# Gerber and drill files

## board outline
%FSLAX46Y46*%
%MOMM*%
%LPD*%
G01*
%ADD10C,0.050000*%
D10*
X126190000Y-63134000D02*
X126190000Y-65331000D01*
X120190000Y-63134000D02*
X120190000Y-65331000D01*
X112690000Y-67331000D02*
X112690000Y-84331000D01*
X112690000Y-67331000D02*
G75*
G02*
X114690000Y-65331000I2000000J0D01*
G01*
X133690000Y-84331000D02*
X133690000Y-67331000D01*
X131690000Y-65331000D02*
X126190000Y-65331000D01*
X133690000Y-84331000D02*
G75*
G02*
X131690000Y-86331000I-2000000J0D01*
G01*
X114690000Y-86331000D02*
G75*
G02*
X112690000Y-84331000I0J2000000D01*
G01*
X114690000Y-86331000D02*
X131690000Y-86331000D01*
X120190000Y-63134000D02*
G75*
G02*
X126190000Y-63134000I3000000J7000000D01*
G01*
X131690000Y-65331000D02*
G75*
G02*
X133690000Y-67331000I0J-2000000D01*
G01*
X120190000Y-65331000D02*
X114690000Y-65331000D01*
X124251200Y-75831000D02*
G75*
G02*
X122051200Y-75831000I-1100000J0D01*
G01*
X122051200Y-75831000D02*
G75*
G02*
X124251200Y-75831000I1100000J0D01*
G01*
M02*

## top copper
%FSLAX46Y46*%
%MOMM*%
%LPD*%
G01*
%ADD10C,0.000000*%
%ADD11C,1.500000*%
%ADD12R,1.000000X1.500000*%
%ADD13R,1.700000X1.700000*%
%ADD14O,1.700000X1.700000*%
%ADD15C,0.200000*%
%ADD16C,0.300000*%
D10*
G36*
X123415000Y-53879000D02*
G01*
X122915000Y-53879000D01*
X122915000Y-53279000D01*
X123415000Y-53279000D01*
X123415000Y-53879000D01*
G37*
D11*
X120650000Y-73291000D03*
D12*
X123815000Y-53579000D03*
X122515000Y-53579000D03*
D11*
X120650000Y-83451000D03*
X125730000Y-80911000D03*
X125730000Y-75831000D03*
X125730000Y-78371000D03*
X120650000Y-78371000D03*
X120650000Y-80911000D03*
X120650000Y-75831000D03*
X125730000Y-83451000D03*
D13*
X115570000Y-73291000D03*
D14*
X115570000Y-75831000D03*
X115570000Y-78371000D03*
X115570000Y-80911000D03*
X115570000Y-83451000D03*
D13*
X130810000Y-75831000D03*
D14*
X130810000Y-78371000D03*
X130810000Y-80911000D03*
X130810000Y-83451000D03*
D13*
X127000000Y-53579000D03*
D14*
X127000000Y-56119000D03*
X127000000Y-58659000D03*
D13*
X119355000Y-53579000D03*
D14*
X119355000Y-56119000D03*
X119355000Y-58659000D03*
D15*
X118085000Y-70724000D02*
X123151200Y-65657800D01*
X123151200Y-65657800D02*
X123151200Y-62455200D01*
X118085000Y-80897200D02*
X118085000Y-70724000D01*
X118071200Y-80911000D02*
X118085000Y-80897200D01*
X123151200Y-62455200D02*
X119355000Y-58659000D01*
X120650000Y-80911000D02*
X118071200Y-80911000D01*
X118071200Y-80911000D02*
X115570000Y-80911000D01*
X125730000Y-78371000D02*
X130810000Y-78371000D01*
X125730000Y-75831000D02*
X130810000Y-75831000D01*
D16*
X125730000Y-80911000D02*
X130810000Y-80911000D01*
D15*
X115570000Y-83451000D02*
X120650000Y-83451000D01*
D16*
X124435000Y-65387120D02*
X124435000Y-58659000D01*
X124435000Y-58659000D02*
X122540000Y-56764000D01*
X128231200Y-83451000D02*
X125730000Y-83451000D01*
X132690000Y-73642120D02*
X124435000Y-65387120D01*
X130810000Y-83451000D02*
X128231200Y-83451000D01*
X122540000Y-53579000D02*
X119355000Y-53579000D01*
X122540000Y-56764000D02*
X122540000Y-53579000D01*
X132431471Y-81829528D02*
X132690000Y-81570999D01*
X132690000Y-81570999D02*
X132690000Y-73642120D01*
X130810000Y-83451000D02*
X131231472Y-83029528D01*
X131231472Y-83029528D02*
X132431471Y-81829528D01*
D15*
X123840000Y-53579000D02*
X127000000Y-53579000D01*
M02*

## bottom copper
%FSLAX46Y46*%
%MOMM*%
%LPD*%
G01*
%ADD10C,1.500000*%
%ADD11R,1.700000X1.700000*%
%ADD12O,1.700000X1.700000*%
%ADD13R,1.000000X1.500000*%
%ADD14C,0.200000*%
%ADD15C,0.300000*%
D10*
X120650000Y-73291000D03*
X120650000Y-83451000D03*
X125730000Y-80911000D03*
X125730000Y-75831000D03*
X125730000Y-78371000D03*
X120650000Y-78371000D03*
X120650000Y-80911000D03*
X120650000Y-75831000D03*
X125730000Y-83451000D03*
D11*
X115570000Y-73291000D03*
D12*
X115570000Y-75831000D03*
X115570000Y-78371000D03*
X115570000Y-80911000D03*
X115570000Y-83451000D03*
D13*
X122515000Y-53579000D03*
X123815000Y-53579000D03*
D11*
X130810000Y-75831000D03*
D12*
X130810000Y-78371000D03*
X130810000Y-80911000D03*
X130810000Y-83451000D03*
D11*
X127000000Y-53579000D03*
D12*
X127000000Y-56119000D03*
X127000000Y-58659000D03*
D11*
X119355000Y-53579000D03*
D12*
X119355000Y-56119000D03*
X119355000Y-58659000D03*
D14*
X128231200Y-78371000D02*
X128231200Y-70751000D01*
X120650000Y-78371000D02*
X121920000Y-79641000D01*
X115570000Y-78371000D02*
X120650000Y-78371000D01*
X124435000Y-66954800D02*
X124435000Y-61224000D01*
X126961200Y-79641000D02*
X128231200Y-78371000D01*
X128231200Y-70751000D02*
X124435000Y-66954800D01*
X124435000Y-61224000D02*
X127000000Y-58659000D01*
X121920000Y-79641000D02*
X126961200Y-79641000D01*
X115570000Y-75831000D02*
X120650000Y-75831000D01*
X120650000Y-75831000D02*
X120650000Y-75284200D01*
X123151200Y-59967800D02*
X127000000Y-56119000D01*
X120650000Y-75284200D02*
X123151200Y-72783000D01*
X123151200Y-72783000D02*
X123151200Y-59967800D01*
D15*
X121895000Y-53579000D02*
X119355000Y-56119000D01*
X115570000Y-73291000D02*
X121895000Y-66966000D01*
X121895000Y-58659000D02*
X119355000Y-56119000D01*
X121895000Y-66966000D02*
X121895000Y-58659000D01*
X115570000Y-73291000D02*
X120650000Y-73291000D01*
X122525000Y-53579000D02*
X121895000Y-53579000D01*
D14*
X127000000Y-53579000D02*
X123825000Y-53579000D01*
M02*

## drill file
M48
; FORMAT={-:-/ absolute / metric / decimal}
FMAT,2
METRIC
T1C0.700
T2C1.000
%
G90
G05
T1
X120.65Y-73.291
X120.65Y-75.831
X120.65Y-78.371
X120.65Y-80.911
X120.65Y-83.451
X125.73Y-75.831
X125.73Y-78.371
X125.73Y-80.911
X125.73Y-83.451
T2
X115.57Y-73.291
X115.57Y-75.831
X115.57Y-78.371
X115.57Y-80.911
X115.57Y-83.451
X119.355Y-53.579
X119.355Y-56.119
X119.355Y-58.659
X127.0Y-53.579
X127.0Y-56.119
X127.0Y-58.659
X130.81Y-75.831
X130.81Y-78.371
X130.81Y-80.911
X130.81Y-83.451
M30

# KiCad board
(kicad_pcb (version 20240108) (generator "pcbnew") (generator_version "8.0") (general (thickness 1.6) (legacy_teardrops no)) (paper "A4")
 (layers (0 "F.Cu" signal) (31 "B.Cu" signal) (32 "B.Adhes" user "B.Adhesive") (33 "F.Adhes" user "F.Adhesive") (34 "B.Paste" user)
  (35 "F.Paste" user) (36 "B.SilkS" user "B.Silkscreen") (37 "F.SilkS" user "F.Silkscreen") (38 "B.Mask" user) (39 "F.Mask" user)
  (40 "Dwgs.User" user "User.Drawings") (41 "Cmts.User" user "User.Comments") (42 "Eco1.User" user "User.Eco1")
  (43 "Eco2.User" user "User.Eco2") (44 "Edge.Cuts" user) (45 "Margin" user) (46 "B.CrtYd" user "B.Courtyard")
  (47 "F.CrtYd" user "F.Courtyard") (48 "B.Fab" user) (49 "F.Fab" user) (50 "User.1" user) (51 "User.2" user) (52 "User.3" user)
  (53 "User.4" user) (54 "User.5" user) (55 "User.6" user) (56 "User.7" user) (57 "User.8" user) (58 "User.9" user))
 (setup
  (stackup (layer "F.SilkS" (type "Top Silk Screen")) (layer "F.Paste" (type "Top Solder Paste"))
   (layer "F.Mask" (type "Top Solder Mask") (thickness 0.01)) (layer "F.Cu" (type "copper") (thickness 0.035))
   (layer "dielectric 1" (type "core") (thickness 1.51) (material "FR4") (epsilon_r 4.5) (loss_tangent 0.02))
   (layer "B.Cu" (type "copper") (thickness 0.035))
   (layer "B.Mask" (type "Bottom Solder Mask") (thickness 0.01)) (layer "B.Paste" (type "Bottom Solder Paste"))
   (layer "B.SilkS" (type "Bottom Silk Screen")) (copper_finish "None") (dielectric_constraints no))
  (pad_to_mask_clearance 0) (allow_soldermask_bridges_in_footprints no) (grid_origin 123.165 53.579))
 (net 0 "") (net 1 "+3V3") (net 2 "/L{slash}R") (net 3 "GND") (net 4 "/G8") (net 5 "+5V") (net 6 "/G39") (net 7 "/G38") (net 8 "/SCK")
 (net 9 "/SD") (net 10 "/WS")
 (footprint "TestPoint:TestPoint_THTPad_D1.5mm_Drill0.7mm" (layer "F.Cu") (at 120.65 73.291)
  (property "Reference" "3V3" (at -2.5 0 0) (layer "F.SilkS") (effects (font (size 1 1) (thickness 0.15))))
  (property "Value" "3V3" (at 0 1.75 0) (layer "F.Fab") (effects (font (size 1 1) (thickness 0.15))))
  (pad "1" thru_hole circle (at 0 0) (size 1.5 1.5) (drill 0.7) (layers "*.Cu" "*.Mask") (remove_unused_layers no) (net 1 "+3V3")))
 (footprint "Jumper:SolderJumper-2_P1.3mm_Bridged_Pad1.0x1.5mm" (layer "F.Cu") (at 123.165 53.579 180)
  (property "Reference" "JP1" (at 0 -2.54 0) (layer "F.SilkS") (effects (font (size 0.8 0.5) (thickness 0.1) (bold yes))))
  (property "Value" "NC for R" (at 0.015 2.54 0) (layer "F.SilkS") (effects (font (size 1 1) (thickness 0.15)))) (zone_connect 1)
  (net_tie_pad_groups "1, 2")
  (fp_poly (pts (xy -0.25 -0.3) (xy 0.25 -0.3) (xy 0.25 0.3) (xy -0.25 0.3)) (stroke (width 0) (type solid)) (fill solid) (layer "F.Cu"))
  (pad "1" smd rect (at -0.65 0 180) (size 1 1.5) (layers "F.Cu" "F.Mask") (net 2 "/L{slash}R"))
  (pad "2" smd rect (at 0.65 0 180) (size 1 1.5) (layers "F.Cu" "F.Mask") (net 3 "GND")))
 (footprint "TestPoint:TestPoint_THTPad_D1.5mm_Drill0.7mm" (layer "F.Cu") (at 120.65 83.451)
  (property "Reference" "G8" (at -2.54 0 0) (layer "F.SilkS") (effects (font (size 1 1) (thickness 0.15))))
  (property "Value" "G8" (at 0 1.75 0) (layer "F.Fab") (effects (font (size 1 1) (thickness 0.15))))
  (pad "1" thru_hole circle (at 0 0) (size 1.5 1.5) (drill 0.7) (layers "*.Cu" "*.Mask") (remove_unused_layers no) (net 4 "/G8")))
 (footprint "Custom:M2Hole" (layer "F.Cu") (at 123.1512 75.831)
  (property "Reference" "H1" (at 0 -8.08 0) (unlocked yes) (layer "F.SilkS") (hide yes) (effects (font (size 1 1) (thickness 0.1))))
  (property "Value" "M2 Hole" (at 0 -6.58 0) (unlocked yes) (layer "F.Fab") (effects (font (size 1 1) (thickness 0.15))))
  (fp_circle (center 0 0) (end 1.1 0) (stroke (width 0.05) (type default)) (fill none) (layer "Edge.Cuts")))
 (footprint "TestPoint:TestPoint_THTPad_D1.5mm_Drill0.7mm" (layer "F.Cu") (at 125.73 80.911)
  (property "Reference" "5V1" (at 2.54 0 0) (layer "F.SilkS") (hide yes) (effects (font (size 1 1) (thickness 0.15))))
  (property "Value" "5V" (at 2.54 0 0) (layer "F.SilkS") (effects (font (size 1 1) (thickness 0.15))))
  (pad "1" thru_hole circle (at 0 0) (size 1.5 1.5) (drill 0.7) (layers "*.Cu" "*.Mask") (remove_unused_layers no) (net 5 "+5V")))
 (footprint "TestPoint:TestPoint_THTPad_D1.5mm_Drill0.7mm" (layer "F.Cu") (at 125.73 75.831)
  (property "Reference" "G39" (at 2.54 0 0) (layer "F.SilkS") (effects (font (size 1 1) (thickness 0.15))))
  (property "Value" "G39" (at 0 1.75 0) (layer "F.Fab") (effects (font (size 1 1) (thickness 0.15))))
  (pad "1" thru_hole circle (at 0 0) (size 1.5 1.5) (drill 0.7) (layers "*.Cu" "*.Mask") (remove_unused_layers no) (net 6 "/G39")))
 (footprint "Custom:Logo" (layer "F.Cu") (at 130.01 70.866)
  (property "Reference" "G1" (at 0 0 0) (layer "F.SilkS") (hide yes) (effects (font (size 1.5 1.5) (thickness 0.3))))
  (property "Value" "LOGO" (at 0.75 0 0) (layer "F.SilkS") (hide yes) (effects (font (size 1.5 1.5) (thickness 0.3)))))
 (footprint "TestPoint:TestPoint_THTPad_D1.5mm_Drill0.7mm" (layer "F.Cu") (at 125.73 78.371)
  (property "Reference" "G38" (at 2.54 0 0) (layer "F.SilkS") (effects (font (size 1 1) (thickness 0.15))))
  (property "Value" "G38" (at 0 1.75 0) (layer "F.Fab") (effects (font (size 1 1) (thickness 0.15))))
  (pad "1" thru_hole circle (at 0 0) (size 1.5 1.5) (drill 0.7) (layers "*.Cu" "*.Mask") (remove_unused_layers no) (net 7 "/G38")))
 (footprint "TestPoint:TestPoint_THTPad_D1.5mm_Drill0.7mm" (layer "F.Cu") (at 120.65 78.371)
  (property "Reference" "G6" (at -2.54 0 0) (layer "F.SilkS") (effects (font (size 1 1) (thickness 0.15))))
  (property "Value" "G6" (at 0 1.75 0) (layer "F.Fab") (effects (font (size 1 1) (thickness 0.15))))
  (pad "1" thru_hole circle (at 0 0) (size 1.5 1.5) (drill 0.7) (layers "*.Cu" "*.Mask") (remove_unused_layers no) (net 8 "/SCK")))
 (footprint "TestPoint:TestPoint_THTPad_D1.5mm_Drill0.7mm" (layer "F.Cu") (at 120.65 80.911)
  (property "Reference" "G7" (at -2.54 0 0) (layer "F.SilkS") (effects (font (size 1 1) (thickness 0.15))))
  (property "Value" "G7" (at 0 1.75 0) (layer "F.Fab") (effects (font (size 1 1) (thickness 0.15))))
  (pad "1" thru_hole circle (at 0 0) (size 1.5 1.5) (drill 0.7) (layers "*.Cu" "*.Mask") (remove_unused_layers no) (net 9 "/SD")))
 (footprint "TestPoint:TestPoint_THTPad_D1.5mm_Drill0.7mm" (layer "F.Cu") (at 120.65 75.831)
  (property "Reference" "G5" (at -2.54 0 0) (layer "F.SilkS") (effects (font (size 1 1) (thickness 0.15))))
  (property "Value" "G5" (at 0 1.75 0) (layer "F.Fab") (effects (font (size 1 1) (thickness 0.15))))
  (pad "1" thru_hole circle (at 0 0) (size 1.5 1.5) (drill 0.7) (layers "*.Cu" "*.Mask") (remove_unused_layers no) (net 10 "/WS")))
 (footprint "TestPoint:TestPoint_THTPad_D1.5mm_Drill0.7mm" (layer "F.Cu") (at 125.73 83.451)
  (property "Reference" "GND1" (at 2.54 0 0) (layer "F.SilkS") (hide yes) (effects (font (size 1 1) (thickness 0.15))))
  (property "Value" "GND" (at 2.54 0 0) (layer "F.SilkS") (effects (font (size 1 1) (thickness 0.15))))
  (pad "1" thru_hole circle (at 0 0) (size 1.5 1.5) (drill 0.7) (layers "*.Cu" "*.Mask") (remove_unused_layers no) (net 3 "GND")))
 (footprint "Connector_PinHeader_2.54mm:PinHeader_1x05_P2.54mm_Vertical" (layer "B.Cu") (at 115.57 73.291 180)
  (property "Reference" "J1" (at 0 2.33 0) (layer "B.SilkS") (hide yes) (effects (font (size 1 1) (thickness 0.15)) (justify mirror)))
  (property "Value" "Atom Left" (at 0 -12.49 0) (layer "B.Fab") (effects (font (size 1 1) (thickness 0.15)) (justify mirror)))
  (pad "1" thru_hole rect (at 0 0 180) (size 1.7 1.7) (drill 1) (layers "*.Cu" "*.Mask") (remove_unused_layers no) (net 1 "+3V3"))
  (pad "2" thru_hole oval (at 0 -2.54 180) (size 1.7 1.7) (drill 1) (layers "*.Cu" "*.Mask") (remove_unused_layers no) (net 10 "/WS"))
  (pad "3" thru_hole oval (at 0 -5.08 180) (size 1.7 1.7) (drill 1) (layers "*.Cu" "*.Mask") (remove_unused_layers no) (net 8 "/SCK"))
  (pad "4" thru_hole oval (at 0 -7.62 180) (size 1.7 1.7) (drill 1) (layers "*.Cu" "*.Mask") (remove_unused_layers no) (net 9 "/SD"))
  (pad "5" thru_hole oval (at 0 -10.16 180) (size 1.7 1.7) (drill 1) (layers "*.Cu" "*.Mask") (remove_unused_layers no) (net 4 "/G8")))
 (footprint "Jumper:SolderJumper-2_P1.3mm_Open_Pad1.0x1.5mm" (layer "B.Cu") (at 123.165 53.579)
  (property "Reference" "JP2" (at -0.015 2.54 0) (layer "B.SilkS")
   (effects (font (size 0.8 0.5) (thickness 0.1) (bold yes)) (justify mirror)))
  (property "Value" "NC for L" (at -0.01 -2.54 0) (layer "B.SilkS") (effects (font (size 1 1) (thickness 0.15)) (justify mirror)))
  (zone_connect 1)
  (pad "1" smd rect (at -0.65 0) (size 1 1.5) (layers "B.Cu" "B.Mask") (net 1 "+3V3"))
  (pad "2" smd rect (at 0.65 0) (size 1 1.5) (layers "B.Cu" "B.Mask") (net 2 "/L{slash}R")))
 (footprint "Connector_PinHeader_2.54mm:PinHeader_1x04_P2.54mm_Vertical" (layer "B.Cu") (at 130.81 75.831 180)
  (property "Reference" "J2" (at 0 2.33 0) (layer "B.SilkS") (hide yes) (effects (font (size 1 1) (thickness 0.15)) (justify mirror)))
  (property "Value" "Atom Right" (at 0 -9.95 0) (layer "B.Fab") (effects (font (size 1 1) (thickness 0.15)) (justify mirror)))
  (pad "1" thru_hole rect (at 0 0 180) (size 1.7 1.7) (drill 1) (layers "*.Cu" "*.Mask") (remove_unused_layers no) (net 6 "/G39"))
  (pad "2" thru_hole oval (at 0 -2.54 180) (size 1.7 1.7) (drill 1) (layers "*.Cu" "*.Mask") (remove_unused_layers no) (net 7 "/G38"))
  (pad "3" thru_hole oval (at 0 -5.08 180) (size 1.7 1.7) (drill 1) (layers "*.Cu" "*.Mask") (remove_unused_layers no) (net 5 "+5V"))
  (pad "4" thru_hole oval (at 0 -7.62 180) (size 1.7 1.7) (drill 1) (layers "*.Cu" "*.Mask") (remove_unused_layers no) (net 3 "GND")))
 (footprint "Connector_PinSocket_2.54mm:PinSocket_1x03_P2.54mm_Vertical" (layer "B.Cu") (at 127 53.579 180)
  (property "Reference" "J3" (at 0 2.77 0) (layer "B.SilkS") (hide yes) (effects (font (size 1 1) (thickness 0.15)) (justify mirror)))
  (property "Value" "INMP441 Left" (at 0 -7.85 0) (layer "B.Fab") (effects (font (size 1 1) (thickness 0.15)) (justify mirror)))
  (pad "1" thru_hole rect (at 0 0 180) (size 1.7 1.7) (drill 1) (layers "*.Cu" "*.Mask") (remove_unused_layers no) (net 2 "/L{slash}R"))
  (pad "2" thru_hole oval (at 0 -2.54 180) (size 1.7 1.7) (drill 1) (layers "*.Cu" "*.Mask") (remove_unused_layers no) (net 10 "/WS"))
  (pad "3" thru_hole oval (at 0 -5.08 180) (size 1.7 1.7) (drill 1) (layers "*.Cu" "*.Mask") (remove_unused_layers no) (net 8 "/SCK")))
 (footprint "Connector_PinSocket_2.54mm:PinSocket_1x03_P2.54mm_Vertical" (layer "B.Cu") (at 119.355 53.579 180)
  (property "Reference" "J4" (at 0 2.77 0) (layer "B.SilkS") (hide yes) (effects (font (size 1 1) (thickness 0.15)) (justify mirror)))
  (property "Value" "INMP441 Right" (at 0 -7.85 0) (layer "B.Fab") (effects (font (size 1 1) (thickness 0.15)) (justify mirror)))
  (pad "1" thru_hole rect (at 0 0 180) (size 1.7 1.7) (drill 1) (layers "*.Cu" "*.Mask") (remove_unused_layers no) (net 3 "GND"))
  (pad "2" thru_hole oval (at 0 -2.54 180) (size 1.7 1.7) (drill 1) (layers "*.Cu" "*.Mask") (remove_unused_layers no) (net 1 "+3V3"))
  (pad "3" thru_hole oval (at 0 -5.08 180) (size 1.7 1.7) (drill 1) (layers "*.Cu" "*.Mask") (remove_unused_layers no) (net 9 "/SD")))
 (gr_line (start 126.19 63.134) (end 126.19 65.331) (stroke (width 0.05) (type default)) (layer "Edge.Cuts"))
 (gr_line (start 120.19 63.134) (end 120.19 65.331) (stroke (width 0.05) (type default)) (layer "Edge.Cuts"))
 (gr_line (start 112.69 67.331) (end 112.69 84.331) (stroke (width 0.05) (type default)) (layer "Edge.Cuts"))
 (gr_arc (start 112.69 67.331) (mid 113.275786 65.916786) (end 114.69 65.331) (stroke (width 0.05) (type default)) (layer "Edge.Cuts"))
 (gr_line (start 133.69 84.331) (end 133.69 67.331) (stroke (width 0.05) (type default)) (layer "Edge.Cuts"))
 (gr_line (start 131.69 65.331) (end 126.19 65.331) (stroke (width 0.05) (type default)) (layer "Edge.Cuts"))
 (gr_arc (start 133.69 84.331) (mid 133.104214 85.745214) (end 131.69 86.331) (stroke (width 0.05) (type default)) (layer "Edge.Cuts"))
 (gr_arc (start 114.69 86.331) (mid 113.275786 85.745214) (end 112.69 84.331) (stroke (width 0.05) (type default)) (layer "Edge.Cuts"))
 (gr_line (start 114.69 86.331) (end 131.69 86.331) (stroke (width 0.05) (type default)) (layer "Edge.Cuts"))
 (gr_arc (start 120.19 63.134) (mid 123.19 48.518227) (end 126.19 63.134) (stroke (width 0.05) (type default)) (layer "Edge.Cuts"))
 (gr_arc (start 131.69 65.331) (mid 133.104214 65.916786) (end 133.69 67.331) (stroke (width 0.05) (type default)) (layer "Edge.Cuts"))
 (gr_line (start 120.19 65.331) (end 114.69 65.331) (stroke (width 0.05) (type default)) (layer "Edge.Cuts"))
 (segment (start 128.2312 78.371) (end 128.2312 70.751) (width 0.2) (layer "B.Cu") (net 8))
 (segment (start 120.65 78.371) (end 121.92 79.641) (width 0.2) (layer "B.Cu") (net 8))
 (segment (start 115.57 78.371) (end 120.65 78.371) (width 0.2) (layer "B.Cu") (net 8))
 (segment (start 124.435 66.9548) (end 124.435 61.224) (width 0.2) (layer "B.Cu") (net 8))
 (segment (start 126.9612 79.641) (end 128.2312 78.371) (width 0.2) (layer "B.Cu") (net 8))
 (segment (start 128.2312 70.751) (end 124.435 66.9548) (width 0.2) (layer "B.Cu") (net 8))
 (segment (start 124.435 61.224) (end 127 58.659) (width 0.2) (layer "B.Cu") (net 8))
 (segment (start 121.92 79.641) (end 126.9612 79.641) (width 0.2) (layer "B.Cu") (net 8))
 (segment (start 115.57 75.831) (end 120.65 75.831) (width 0.2) (layer "B.Cu") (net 10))
 (segment (start 120.65 75.831) (end 120.65 75.2842) (width 0.2) (layer "B.Cu") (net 10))
 (segment (start 123.1512 59.9678) (end 127 56.119) (width 0.2) (layer "B.Cu") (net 10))
 (segment (start 120.65 75.2842) (end 123.1512 72.783) (width 0.2) (layer "B.Cu") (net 10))
 (segment (start 123.1512 72.783) (end 123.1512 59.9678) (width 0.2) (layer "B.Cu") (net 10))
 (segment (start 118.085 70.724) (end 123.1512 65.6578) (width 0.2) (layer "F.Cu") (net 9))
 (segment (start 123.1512 65.6578) (end 123.1512 62.4552) (width 0.2) (layer "F.Cu") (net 9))
 (segment (start 118.085 80.8972) (end 118.085 70.724) (width 0.2) (layer "F.Cu") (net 9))
 (segment (start 118.0712 80.911) (end 118.085 80.8972) (width 0.2) (layer "F.Cu") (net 9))
 (segment (start 123.1512 62.4552) (end 119.355 58.659) (width 0.2) (layer "F.Cu") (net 9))
 (segment (start 120.65 80.911) (end 118.0712 80.911) (width 0.2) (layer "F.Cu") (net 9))
 (segment (start 118.0712 80.911) (end 115.57 80.911) (width 0.2) (layer "F.Cu") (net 9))
 (segment (start 121.895 53.579) (end 119.355 56.119) (width 0.3) (layer "B.Cu") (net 1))
 (segment (start 115.57 73.291) (end 121.895 66.966) (width 0.3) (layer "B.Cu") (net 1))
 (segment (start 121.895 58.659) (end 119.355 56.119) (width 0.3) (layer "B.Cu") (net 1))
 (segment (start 121.895 66.966) (end 121.895 58.659) (width 0.3) (layer "B.Cu") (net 1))
 (segment (start 115.57 73.291) (end 120.65 73.291) (width 0.3) (layer "B.Cu") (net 1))
 (segment (start 122.525 53.579) (end 121.895 53.579) (width 0.3) (layer "B.Cu") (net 1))
 (segment (start 125.73 78.371) (end 130.81 78.371) (width 0.2) (layer "F.Cu") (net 7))
 (segment (start 125.73 75.831) (end 130.81 75.831) (width 0.2) (layer "F.Cu") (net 6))
 (segment (start 125.73 80.911) (end 130.81 80.911) (width 0.3) (layer "F.Cu") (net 5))
 (segment (start 115.57 83.451) (end 120.65 83.451) (width 0.2) (layer "F.Cu") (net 4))
 (segment (start 124.435 65.38712) (end 124.435 58.659) (width 0.3) (layer "F.Cu") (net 3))
 (segment (start 124.435 58.659) (end 122.54 56.764) (width 0.3) (layer "F.Cu") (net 3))
 (segment (start 128.2312 83.451) (end 125.73 83.451) (width 0.3) (layer "F.Cu") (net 3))
 (segment (start 132.69 73.64212) (end 124.435 65.38712) (width 0.3) (layer "F.Cu") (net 3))
 (segment (start 130.81 83.451) (end 128.2312 83.451) (width 0.3) (layer "F.Cu") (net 3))
 (segment (start 122.54 53.579) (end 119.355 53.579) (width 0.3) (layer "F.Cu") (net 3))
 (segment (start 122.54 56.764) (end 122.54 53.579) (width 0.3) (layer "F.Cu") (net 3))
 (segment (start 132.431471 81.829528) (end 132.69 81.570999) (width 0.3) (layer "F.Cu") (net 3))
 (segment (start 132.69 81.570999) (end 132.69 73.64212) (width 0.3) (layer "F.Cu") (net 3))
 (segment (start 130.81 83.451) (end 131.231472 83.029528) (width 0.3) (layer "F.Cu") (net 3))
 (segment (start 131.231472 83.029528) (end 132.431471 81.829528) (width 0.3) (layer "F.Cu") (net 3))
 (segment (start 123.84 53.579) (end 127 53.579) (width 0.2) (layer "F.Cu") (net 2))
 (segment (start 127 53.579) (end 123.825 53.579) (width 0.2) (layer "B.Cu") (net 2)))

